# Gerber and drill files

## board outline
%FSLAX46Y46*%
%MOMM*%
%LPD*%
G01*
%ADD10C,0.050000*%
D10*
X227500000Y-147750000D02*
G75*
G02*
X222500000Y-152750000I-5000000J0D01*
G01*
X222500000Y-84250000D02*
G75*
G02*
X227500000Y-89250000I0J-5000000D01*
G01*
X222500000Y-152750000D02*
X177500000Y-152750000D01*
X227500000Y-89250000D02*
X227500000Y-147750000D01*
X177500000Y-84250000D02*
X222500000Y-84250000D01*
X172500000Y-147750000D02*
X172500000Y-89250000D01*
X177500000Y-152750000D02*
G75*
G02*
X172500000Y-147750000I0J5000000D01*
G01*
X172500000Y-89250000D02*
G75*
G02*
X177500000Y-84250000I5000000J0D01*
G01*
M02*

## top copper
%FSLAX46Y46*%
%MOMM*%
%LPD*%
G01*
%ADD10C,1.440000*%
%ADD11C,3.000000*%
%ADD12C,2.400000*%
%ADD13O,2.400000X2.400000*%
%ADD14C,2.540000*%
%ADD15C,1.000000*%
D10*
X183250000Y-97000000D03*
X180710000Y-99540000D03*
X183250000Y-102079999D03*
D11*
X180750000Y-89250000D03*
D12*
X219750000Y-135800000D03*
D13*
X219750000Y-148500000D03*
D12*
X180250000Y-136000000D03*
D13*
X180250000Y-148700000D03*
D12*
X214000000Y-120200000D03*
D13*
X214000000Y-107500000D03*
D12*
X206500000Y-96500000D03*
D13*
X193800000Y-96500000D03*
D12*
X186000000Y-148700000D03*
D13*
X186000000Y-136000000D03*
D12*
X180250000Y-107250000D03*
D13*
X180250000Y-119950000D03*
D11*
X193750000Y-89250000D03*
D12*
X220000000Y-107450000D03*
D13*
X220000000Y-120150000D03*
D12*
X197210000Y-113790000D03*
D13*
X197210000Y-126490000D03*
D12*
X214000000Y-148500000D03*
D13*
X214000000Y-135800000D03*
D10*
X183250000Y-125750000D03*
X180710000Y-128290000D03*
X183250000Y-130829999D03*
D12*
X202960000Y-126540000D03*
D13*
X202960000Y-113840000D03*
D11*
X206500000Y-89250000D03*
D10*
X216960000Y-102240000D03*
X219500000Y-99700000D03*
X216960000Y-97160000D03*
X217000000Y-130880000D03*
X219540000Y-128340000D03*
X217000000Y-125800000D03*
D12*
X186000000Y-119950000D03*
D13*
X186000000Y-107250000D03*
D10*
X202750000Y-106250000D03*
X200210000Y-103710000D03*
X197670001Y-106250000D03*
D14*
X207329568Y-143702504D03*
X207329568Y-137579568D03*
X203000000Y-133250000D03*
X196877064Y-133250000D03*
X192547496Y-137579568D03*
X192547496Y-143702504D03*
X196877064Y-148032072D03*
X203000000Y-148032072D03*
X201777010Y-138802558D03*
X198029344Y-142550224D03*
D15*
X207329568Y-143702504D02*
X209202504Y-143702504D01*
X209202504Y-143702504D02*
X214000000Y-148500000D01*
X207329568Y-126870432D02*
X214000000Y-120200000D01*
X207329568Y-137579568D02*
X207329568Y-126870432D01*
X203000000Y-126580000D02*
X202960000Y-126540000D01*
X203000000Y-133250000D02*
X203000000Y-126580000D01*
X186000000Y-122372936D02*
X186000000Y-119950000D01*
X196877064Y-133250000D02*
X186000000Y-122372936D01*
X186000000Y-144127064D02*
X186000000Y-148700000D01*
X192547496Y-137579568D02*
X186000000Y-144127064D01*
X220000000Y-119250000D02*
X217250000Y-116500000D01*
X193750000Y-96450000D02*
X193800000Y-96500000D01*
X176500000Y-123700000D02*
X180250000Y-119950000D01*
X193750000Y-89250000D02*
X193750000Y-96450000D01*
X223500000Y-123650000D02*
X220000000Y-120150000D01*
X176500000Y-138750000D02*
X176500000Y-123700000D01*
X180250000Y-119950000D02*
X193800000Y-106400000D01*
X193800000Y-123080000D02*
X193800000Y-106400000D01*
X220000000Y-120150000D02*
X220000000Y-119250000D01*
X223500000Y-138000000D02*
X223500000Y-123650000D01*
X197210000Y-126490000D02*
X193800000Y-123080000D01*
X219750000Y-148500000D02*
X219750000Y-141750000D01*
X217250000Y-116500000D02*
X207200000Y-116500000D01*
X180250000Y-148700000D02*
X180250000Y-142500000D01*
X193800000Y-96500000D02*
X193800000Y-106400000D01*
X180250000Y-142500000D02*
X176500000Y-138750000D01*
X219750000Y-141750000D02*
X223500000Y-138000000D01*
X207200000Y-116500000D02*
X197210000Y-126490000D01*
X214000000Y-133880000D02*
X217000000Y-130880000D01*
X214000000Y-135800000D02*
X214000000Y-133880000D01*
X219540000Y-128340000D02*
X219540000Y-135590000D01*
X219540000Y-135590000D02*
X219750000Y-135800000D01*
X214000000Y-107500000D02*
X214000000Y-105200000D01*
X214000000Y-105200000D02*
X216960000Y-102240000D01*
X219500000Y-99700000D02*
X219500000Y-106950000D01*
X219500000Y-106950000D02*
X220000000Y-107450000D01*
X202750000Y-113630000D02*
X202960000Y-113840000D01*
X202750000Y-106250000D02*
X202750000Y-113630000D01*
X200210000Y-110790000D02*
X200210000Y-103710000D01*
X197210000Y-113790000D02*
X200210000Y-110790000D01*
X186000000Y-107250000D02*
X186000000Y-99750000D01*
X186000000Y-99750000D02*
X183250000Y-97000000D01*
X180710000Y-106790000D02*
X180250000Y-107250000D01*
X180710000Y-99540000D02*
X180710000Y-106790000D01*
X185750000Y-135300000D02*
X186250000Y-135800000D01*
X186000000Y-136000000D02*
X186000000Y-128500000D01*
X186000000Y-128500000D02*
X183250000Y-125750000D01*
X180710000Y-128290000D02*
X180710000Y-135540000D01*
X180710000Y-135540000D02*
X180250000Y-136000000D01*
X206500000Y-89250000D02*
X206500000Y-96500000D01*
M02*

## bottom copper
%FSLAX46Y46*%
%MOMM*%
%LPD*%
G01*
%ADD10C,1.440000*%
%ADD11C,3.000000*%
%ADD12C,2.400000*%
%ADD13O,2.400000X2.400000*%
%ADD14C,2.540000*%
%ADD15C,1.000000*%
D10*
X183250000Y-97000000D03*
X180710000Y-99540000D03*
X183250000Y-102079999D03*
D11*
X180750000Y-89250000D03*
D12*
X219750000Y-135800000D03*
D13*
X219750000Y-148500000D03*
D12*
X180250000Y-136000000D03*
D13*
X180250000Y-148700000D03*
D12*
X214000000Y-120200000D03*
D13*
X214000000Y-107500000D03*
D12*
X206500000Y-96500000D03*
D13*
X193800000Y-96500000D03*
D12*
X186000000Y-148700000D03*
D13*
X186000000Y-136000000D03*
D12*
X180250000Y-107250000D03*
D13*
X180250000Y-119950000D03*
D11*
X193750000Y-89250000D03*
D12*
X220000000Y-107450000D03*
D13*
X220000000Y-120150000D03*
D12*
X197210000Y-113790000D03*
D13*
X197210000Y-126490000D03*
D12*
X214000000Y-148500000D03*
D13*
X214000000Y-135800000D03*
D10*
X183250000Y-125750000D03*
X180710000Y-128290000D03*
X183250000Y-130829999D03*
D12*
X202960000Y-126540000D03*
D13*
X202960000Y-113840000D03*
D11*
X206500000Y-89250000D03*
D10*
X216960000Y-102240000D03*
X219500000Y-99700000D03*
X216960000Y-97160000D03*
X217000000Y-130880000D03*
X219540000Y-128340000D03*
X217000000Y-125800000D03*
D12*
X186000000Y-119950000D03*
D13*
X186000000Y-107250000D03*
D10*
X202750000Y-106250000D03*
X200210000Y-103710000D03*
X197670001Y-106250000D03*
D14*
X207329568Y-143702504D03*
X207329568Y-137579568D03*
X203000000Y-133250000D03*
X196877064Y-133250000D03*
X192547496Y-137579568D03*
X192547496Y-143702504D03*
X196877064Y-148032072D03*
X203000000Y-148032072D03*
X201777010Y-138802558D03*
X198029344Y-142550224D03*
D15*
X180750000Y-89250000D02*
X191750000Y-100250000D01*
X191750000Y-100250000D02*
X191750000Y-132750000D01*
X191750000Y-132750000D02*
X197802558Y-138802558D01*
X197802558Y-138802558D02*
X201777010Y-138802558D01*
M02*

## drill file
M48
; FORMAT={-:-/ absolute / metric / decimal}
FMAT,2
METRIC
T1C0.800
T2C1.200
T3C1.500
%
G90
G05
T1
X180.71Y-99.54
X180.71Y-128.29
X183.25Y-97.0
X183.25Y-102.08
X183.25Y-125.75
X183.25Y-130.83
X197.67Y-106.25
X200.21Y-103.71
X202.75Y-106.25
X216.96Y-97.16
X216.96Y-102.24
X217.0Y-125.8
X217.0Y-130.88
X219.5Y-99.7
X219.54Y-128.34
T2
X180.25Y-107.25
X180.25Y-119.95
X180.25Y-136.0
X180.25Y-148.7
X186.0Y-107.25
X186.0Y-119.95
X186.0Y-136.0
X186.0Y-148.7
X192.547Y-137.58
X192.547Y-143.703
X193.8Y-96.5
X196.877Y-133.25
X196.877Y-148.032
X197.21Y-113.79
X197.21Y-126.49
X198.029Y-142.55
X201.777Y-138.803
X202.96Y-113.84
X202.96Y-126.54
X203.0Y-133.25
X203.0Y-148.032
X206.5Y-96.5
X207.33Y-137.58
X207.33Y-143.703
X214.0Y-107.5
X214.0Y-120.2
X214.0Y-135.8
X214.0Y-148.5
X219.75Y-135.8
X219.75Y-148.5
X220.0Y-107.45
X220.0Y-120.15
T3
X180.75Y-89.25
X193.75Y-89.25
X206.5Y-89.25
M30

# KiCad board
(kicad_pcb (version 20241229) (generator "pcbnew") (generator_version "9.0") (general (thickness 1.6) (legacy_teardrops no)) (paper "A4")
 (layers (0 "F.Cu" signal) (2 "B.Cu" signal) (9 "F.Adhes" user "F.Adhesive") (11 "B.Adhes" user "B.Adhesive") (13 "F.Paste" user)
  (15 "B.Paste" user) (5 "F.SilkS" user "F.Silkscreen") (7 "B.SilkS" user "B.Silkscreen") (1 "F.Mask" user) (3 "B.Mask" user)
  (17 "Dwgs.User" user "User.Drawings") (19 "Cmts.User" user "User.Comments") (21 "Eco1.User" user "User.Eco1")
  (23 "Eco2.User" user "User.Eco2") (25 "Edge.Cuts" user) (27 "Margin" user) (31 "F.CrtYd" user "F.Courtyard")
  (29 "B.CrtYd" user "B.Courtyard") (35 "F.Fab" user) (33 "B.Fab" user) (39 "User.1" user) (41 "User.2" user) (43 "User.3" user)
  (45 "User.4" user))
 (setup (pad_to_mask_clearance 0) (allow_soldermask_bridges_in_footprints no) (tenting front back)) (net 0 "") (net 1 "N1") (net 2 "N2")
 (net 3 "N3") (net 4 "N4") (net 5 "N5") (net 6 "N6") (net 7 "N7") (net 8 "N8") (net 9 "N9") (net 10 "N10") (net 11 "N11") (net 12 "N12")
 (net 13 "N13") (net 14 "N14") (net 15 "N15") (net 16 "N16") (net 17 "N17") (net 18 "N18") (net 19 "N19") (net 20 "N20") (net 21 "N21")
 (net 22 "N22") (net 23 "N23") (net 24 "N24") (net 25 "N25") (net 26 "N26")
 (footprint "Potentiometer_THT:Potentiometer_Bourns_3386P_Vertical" (layer "F.Cu") (at 183.25 97 180)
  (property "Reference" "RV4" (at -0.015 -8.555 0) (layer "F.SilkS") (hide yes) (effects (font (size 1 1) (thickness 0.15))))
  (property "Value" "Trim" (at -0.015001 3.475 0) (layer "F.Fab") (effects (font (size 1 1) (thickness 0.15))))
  (pad "1" thru_hole circle (at 0 0 180) (size 1.44 1.44) (drill 0.8) (layers "*.Cu" "*.Mask") (remove_unused_layers no) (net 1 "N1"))
  (pad "2" thru_hole circle (at 2.54 -2.54 180) (size 1.44 1.44) (drill 0.8) (layers "*.Cu" "*.Mask") (remove_unused_layers no) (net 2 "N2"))
  (pad "3" thru_hole circle (at 0 -5.079999 180) (size 1.44 1.44) (drill 0.8) (layers "*.Cu" "*.Mask") (remove_unused_layers no)
   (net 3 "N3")))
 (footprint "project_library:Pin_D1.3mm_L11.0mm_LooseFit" (layer "F.Cu") (at 180.75 89.25)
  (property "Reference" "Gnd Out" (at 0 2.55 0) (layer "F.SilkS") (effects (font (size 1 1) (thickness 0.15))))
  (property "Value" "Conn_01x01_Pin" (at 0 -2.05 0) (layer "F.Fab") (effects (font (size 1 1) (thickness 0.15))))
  (pad "1" thru_hole circle (at 0 0) (size 3 3) (drill 1.5) (layers "*.Cu" "*.Mask") (remove_unused_layers no) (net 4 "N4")))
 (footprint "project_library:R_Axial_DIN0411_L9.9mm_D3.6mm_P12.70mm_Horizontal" (layer "F.Cu") (at 219.75 135.8 -90)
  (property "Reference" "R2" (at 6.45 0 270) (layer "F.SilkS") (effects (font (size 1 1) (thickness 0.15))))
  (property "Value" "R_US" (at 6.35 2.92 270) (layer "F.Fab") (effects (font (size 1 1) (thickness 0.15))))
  (pad "1" thru_hole circle (at 0 0 270) (size 2.4 2.4) (drill 1.2) (layers "*.Cu" "*.Mask") (remove_unused_layers no) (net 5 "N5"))
  (pad "2" thru_hole oval (at 12.7 0 270) (size 2.4 2.4) (drill 1.2) (layers "*.Cu" "*.Mask") (remove_unused_layers no) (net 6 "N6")))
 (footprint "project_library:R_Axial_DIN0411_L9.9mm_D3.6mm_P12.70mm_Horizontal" (layer "F.Cu") (at 180.25 136 -90)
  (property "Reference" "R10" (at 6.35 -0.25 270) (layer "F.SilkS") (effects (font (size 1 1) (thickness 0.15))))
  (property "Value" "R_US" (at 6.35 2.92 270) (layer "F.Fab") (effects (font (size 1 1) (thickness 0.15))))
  (pad "1" thru_hole circle (at 0 0 270) (size 2.4 2.4) (drill 1.2) (layers "*.Cu" "*.Mask") (remove_unused_layers no) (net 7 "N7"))
  (pad "2" thru_hole oval (at 12.7 0 270) (size 2.4 2.4) (drill 1.2) (layers "*.Cu" "*.Mask") (remove_unused_layers no) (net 6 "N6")))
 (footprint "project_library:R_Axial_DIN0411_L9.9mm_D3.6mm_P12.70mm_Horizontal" (layer "F.Cu") (at 214 120.2 90)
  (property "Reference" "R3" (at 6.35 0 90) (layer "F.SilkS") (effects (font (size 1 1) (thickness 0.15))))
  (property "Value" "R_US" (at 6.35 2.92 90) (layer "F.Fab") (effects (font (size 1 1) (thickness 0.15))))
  (pad "1" thru_hole circle (at 0 0 90) (size 2.4 2.4) (drill 1.2) (layers "*.Cu" "*.Mask") (remove_unused_layers no) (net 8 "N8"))
  (pad "2" thru_hole oval (at 12.7 0 90) (size 2.4 2.4) (drill 1.2) (layers "*.Cu" "*.Mask") (remove_unused_layers no) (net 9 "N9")))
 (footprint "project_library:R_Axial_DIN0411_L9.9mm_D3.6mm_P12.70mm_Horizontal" (layer "F.Cu") (at 206.5 96.5 180)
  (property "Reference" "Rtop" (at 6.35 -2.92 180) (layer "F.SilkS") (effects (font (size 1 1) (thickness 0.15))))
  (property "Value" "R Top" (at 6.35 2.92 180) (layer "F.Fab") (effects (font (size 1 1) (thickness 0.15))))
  (pad "1" thru_hole circle (at 0 0 180) (size 2.4 2.4) (drill 1.2) (layers "*.Cu" "*.Mask") (remove_unused_layers no) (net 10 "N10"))
  (pad "2" thru_hole oval (at 12.7 0 180) (size 2.4 2.4) (drill 1.2) (layers "*.Cu" "*.Mask") (remove_unused_layers no) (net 6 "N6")))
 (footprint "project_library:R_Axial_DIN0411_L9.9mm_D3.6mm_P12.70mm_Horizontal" (layer "F.Cu") (at 186 148.7 90)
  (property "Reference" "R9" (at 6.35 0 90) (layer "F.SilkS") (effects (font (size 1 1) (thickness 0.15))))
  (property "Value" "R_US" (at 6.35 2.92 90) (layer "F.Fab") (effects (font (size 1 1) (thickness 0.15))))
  (pad "1" thru_hole circle (at 0 0 90) (size 2.4 2.4) (drill 1.2) (layers "*.Cu" "*.Mask") (remove_unused_layers no) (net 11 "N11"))
  (pad "2" thru_hole oval (at 12.7 0 90) (size 2.4 2.4) (drill 1.2) (layers "*.Cu" "*.Mask") (remove_unused_layers no) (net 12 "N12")))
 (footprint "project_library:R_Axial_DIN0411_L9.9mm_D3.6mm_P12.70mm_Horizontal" (layer "F.Cu") (at 180.25 107.25 -90)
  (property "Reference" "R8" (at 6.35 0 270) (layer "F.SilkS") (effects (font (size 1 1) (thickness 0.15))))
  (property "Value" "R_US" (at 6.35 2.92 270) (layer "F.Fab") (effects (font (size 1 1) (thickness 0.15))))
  (pad "1" thru_hole circle (at 0 0 270) (size 2.4 2.4) (drill 1.2) (layers "*.Cu" "*.Mask") (remove_unused_layers no) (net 2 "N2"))
  (pad "2" thru_hole oval (at 12.7 0 270) (size 2.4 2.4) (drill 1.2) (layers "*.Cu" "*.Mask") (remove_unused_layers no) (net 6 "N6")))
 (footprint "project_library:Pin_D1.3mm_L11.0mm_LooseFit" (layer "F.Cu") (at 193.75 89.25)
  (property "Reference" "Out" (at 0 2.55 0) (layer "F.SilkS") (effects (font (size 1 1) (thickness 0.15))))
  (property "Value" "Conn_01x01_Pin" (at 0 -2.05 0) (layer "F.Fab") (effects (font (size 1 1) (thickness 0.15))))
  (pad "1" thru_hole circle (at 0 0) (size 3 3) (drill 1.5) (layers "*.Cu" "*.Mask") (remove_unused_layers no) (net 6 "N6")))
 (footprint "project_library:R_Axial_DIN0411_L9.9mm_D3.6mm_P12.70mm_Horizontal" (layer "F.Cu") (at 220 107.45 -90)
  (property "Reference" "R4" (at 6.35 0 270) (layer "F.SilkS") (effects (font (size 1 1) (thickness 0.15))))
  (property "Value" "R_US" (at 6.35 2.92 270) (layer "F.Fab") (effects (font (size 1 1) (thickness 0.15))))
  (pad "1" thru_hole circle (at 0 0 270) (size 2.4 2.4) (drill 1.2) (layers "*.Cu" "*.Mask") (remove_unused_layers no) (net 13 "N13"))
  (pad "2" thru_hole oval (at 12.7 0 270) (size 2.4 2.4) (drill 1.2) (layers "*.Cu" "*.Mask") (remove_unused_layers no) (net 6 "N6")))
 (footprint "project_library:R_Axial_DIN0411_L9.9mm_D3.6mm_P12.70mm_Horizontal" (layer "F.Cu") (at 197.21 113.79 -90)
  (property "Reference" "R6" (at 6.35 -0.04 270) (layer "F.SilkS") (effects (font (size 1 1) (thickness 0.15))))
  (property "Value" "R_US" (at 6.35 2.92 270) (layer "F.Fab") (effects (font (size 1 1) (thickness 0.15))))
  (pad "1" thru_hole circle (at 0 0 270) (size 2.4 2.4) (drill 1.2) (layers "*.Cu" "*.Mask") (remove_unused_layers no) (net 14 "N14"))
  (pad "2" thru_hole oval (at 12.7 0 270) (size 2.4 2.4) (drill 1.2) (layers "*.Cu" "*.Mask") (remove_unused_layers no) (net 6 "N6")))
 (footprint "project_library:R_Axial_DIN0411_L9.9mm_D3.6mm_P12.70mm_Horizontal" (layer "F.Cu") (at 214 148.5 90)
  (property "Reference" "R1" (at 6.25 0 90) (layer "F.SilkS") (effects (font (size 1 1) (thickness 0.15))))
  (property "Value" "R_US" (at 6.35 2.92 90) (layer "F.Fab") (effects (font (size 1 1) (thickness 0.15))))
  (pad "1" thru_hole circle (at 0 0 90) (size 2.4 2.4) (drill 1.2) (layers "*.Cu" "*.Mask") (remove_unused_layers no) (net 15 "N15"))
  (pad "2" thru_hole oval (at 12.7 0 90) (size 2.4 2.4) (drill 1.2) (layers "*.Cu" "*.Mask") (remove_unused_layers no) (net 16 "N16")))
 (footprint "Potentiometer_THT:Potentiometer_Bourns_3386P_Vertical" (layer "F.Cu") (at 183.25 125.75 180)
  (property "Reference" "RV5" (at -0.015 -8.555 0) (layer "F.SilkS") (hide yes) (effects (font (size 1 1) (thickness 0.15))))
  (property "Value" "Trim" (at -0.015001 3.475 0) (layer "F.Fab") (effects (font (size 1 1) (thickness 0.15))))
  (pad "1" thru_hole circle (at 0 0 180) (size 1.44 1.44) (drill 0.8) (layers "*.Cu" "*.Mask") (remove_unused_layers no) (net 12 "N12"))
  (pad "2" thru_hole circle (at 2.54 -2.54 180) (size 1.44 1.44) (drill 0.8) (layers "*.Cu" "*.Mask") (remove_unused_layers no) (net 7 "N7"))
  (pad "3" thru_hole circle (at 0 -5.079999 180) (size 1.44 1.44) (drill 0.8) (layers "*.Cu" "*.Mask") (remove_unused_layers no)
   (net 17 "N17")))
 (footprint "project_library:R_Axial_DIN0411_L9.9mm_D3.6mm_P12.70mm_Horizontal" (layer "F.Cu") (at 202.96 126.54 90)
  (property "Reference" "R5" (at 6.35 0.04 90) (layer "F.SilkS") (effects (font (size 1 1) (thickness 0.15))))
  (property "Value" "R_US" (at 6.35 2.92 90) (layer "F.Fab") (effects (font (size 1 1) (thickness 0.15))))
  (pad "1" thru_hole circle (at 0 0 90) (size 2.4 2.4) (drill 1.2) (layers "*.Cu" "*.Mask") (remove_unused_layers no) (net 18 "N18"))
  (pad "2" thru_hole oval (at 12.7 0 90) (size 2.4 2.4) (drill 1.2) (layers "*.Cu" "*.Mask") (remove_unused_layers no) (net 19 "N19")))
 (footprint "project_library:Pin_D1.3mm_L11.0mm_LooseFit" (layer "F.Cu") (at 206.5 89.25)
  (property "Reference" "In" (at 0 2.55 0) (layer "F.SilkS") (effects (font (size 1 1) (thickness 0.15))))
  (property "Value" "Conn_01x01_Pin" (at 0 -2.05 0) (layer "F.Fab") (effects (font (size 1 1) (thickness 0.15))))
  (pad "1" thru_hole circle (at 0 0) (size 3 3) (drill 1.5) (layers "*.Cu" "*.Mask") (remove_unused_layers no) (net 10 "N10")))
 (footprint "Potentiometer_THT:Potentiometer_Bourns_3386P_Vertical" (layer "F.Cu") (at 216.96 102.24)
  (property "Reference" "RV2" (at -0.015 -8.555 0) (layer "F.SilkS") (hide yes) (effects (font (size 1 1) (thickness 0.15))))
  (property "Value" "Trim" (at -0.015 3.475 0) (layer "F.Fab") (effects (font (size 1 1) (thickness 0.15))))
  (pad "1" thru_hole circle (at 0 0) (size 1.44 1.44) (drill 0.8) (layers "*.Cu" "*.Mask") (remove_unused_layers no) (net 9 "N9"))
  (pad "2" thru_hole circle (at 2.54 -2.54) (size 1.44 1.44) (drill 0.8) (layers "*.Cu" "*.Mask") (remove_unused_layers no) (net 13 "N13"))
  (pad "3" thru_hole circle (at 0 -5.08) (size 1.44 1.44) (drill 0.8) (layers "*.Cu" "*.Mask") (remove_unused_layers no) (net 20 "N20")))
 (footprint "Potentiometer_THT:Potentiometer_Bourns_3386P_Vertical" (layer "F.Cu") (at 217 130.88)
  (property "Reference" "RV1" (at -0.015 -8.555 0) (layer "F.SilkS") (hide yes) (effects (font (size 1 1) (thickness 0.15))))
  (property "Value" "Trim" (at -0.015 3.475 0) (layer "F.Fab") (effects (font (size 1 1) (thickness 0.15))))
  (pad "1" thru_hole circle (at 0 0) (size 1.44 1.44) (drill 0.8) (layers "*.Cu" "*.Mask") (remove_unused_layers no) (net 16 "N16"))
  (pad "2" thru_hole circle (at 2.54 -2.54) (size 1.44 1.44) (drill 0.8) (layers "*.Cu" "*.Mask") (remove_unused_layers no) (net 5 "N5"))
  (pad "3" thru_hole circle (at 0 -5.08) (size 1.44 1.44) (drill 0.8) (layers "*.Cu" "*.Mask") (remove_unused_layers no) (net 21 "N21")))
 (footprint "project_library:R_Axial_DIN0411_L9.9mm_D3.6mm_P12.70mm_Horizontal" (layer "F.Cu") (at 186 119.95 90)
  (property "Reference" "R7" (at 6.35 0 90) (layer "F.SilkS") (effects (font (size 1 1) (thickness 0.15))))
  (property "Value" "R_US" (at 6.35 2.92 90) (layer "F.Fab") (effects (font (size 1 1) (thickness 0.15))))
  (pad "1" thru_hole circle (at 0 0 90) (size 2.4 2.4) (drill 1.2) (layers "*.Cu" "*.Mask") (remove_unused_layers no) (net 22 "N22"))
  (pad "2" thru_hole oval (at 12.7 0 90) (size 2.4 2.4) (drill 1.2) (layers "*.Cu" "*.Mask") (remove_unused_layers no) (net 1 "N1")))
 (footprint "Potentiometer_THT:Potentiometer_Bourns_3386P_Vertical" (layer "F.Cu") (at 202.75 106.25 90)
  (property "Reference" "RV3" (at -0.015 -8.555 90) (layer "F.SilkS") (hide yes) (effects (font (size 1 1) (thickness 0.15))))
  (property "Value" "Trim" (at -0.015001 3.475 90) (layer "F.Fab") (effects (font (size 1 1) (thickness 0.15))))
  (pad "1" thru_hole circle (at 0 0 90) (size 1.44 1.44) (drill 0.8) (layers "*.Cu" "*.Mask") (remove_unused_layers no) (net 19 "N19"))
  (pad "2" thru_hole circle (at 2.54 -2.54 90) (size 1.44 1.44) (drill 0.8) (layers "*.Cu" "*.Mask") (remove_unused_layers no)
   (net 14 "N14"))
  (pad "3" thru_hole circle (at 0 -5.079999 90) (size 1.44 1.44) (drill 0.8) (layers "*.Cu" "*.Mask") (remove_unused_layers no)
   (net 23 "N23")))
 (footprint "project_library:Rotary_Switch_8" (layer "B.Cu") (at 199.938532 140.641036 45)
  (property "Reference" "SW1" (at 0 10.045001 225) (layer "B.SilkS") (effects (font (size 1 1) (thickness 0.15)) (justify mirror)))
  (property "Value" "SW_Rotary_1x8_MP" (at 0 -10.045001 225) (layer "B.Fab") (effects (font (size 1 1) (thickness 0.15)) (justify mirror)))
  (pad "1" thru_hole circle (at 3.061467 7.391036 22.5) (size 2.54 2.54) (drill 1.2) (layers "*.Cu" "*.Mask") (remove_unused_layers no)
   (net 15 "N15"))
  (pad "2" thru_hole circle (at 7.391036 3.061467 22.5) (size 2.54 2.54) (drill 1.2) (layers "*.Cu" "*.Mask") (remove_unused_layers no)
   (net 8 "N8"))
  (pad "3" thru_hole circle (at 7.391036 -3.061467 22.5) (size 2.54 2.54) (drill 1.2) (layers "*.Cu" "*.Mask") (remove_unused_layers no)
   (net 18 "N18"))
  (pad "4" thru_hole circle (at 3.061467 -7.391036 22.5) (size 2.54 2.54) (drill 1.2) (layers "*.Cu" "*.Mask") (remove_unused_layers no)
   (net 22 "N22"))
  (pad "5" thru_hole circle (at -3.061467 -7.391036 22.5) (size 2.54 2.54) (drill 1.2) (layers "*.Cu" "*.Mask") (remove_unused_layers no)
   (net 11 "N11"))
  (pad "6" thru_hole circle (at -7.391036 -3.061467 22.5) (size 2.54 2.54) (drill 1.2) (layers "*.Cu" "*.Mask") (remove_unused_layers no)
   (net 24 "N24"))
  (pad "7" thru_hole circle (at -7.391036 3.061467 22.5) (size 2.54 2.54) (drill 1.2) (layers "*.Cu" "*.Mask") (remove_unused_layers no)
   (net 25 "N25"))
  (pad "8" thru_hole circle (at -3.061467 7.391036 22.5) (size 2.54 2.54) (drill 1.2) (layers "*.Cu" "*.Mask") (remove_unused_layers no)
   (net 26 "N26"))
  (pad "9" thru_hole circle (at 2.600001 0 45) (size 2.54 2.54) (drill 1.2) (layers "*.Cu" "*.Mask") (remove_unused_layers no) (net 4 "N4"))
  (pad "MP" thru_hole circle (at -2.7 0 45) (size 2.54 2.54) (drill 1.2) (layers "*.Cu" "*.Mask") (remove_unused_layers no)))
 (gr_arc (start 227.5 147.75) (mid 226.035534 151.285534) (end 222.5 152.75) (stroke (width 0.05) (type default)) (layer "Edge.Cuts"))
 (gr_arc (start 222.5 84.25) (mid 226.035534 85.714466) (end 227.5 89.25) (stroke (width 0.05) (type default)) (layer "Edge.Cuts"))
 (gr_line (start 222.5 152.75) (end 177.5 152.75) (stroke (width 0.05) (type default)) (layer "Edge.Cuts"))
 (gr_line (start 227.5 89.25) (end 227.5 147.75) (stroke (width 0.05) (type default)) (layer "Edge.Cuts"))
 (gr_line (start 177.5 84.25) (end 222.5 84.25) (stroke (width 0.05) (type default)) (layer "Edge.Cuts"))
 (gr_line (start 172.5 147.75) (end 172.5 89.25) (stroke (width 0.05) (type default)) (layer "Edge.Cuts"))
 (gr_arc (start 177.5 152.75) (mid 173.964466 151.285534) (end 172.5 147.75) (stroke (width 0.05) (type default)) (layer "Edge.Cuts"))
 (gr_arc (start 172.5 89.25) (mid 173.964466 85.714466) (end 177.5 84.25) (stroke (width 0.05) (type default)) (layer "Edge.Cuts"))
 (segment (start 207.329568 143.702504) (end 209.202504 143.702504) (width 1) (layer "F.Cu") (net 15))
 (segment (start 209.202504 143.702504) (end 214 148.5) (width 1) (layer "F.Cu") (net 15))
 (segment (start 207.329568 126.870432) (end 214 120.2) (width 1) (layer "F.Cu") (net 8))
 (segment (start 207.329568 137.579568) (end 207.329568 126.870432) (width 1) (layer "F.Cu") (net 8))
 (segment (start 203 126.58) (end 202.96 126.54) (width 1) (layer "F.Cu") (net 18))
 (segment (start 203 133.25) (end 203 126.58) (width 1) (layer "F.Cu") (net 18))
 (segment (start 186 122.372936) (end 186 119.95) (width 1) (layer "F.Cu") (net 22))
 (segment (start 196.877064 133.25) (end 186 122.372936) (width 1) (layer "F.Cu") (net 22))
 (segment (start 186 144.127064) (end 186 148.7) (width 1) (layer "F.Cu") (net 11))
 (segment (start 192.547496 137.579568) (end 186 144.127064) (width 1) (layer "F.Cu") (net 11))
 (segment (start 220 119.25) (end 217.25 116.5) (width 1) (layer "F.Cu") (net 6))
 (segment (start 193.75 96.45) (end 193.8 96.5) (width 1) (layer "F.Cu") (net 6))
 (segment (start 176.5 123.7) (end 180.25 119.95) (width 1) (layer "F.Cu") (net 6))
 (segment (start 193.75 89.25) (end 193.75 96.45) (width 1) (layer "F.Cu") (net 6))
 (segment (start 223.5 123.65) (end 220 120.15) (width 1) (layer "F.Cu") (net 6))
 (segment (start 176.5 138.75) (end 176.5 123.7) (width 1) (layer "F.Cu") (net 6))
 (segment (start 180.25 119.95) (end 193.8 106.4) (width 1) (layer "F.Cu") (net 6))
 (segment (start 193.8 123.08) (end 193.8 106.4) (width 1) (layer "F.Cu") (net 6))
 (segment (start 220 120.15) (end 220 119.25) (width 1) (layer "F.Cu") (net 6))
 (segment (start 223.5 138) (end 223.5 123.65) (width 1) (layer "F.Cu") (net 6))
 (segment (start 197.21 126.49) (end 193.8 123.08) (width 1) (layer "F.Cu") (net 6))
 (segment (start 219.75 148.5) (end 219.75 141.75) (width 1) (layer "F.Cu") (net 6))
 (segment (start 217.25 116.5) (end 207.2 116.5) (width 1) (layer "F.Cu") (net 6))
 (segment (start 180.25 148.7) (end 180.25 142.5) (width 1) (layer "F.Cu") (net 6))
 (segment (start 193.8 96.5) (end 193.8 106.4) (width 1) (layer "F.Cu") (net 6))
 (segment (start 180.25 142.5) (end 176.5 138.75) (width 1) (layer "F.Cu") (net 6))
 (segment (start 219.75 141.75) (end 223.5 138) (width 1) (layer "F.Cu") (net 6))
 (segment (start 207.2 116.5) (end 197.21 126.49) (width 1) (layer "F.Cu") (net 6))
 (segment (start 214 133.88) (end 217 130.88) (width 1) (layer "F.Cu") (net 16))
 (segment (start 214 135.8) (end 214 133.88) (width 1) (layer "F.Cu") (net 16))
 (segment (start 219.54 128.34) (end 219.54 135.59) (width 1) (layer "F.Cu") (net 5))
 (segment (start 219.54 135.59) (end 219.75 135.8) (width 1) (layer "F.Cu") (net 5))
 (segment (start 214 107.5) (end 214 105.2) (width 1) (layer "F.Cu") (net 9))
 (segment (start 214 105.2) (end 216.96 102.24) (width 1) (layer "F.Cu") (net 9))
 (segment (start 219.5 99.7) (end 219.5 106.95) (width 1) (layer "F.Cu") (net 13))
 (segment (start 219.5 106.95) (end 220 107.45) (width 1) (layer "F.Cu") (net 13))
 (segment (start 202.75 113.63) (end 202.96 113.84) (width 1) (layer "F.Cu") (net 19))
 (segment (start 202.75 106.25) (end 202.75 113.63) (width 1) (layer "F.Cu") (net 19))
 (segment (start 200.21 110.79) (end 200.21 103.71) (width 1) (layer "F.Cu") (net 14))
 (segment (start 197.21 113.79) (end 200.21 110.79) (width 1) (layer "F.Cu") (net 14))
 (segment (start 186 107.25) (end 186 99.75) (width 1) (layer "F.Cu") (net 1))
 (segment (start 186 99.75) (end 183.25 97) (width 1) (layer "F.Cu") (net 1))
 (segment (start 180.71 106.79) (end 180.25 107.25) (width 1) (layer "F.Cu") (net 2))
 (segment (start 180.71 99.54) (end 180.71 106.79) (width 1) (layer "F.Cu") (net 2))
 (segment (start 185.75 135.3) (end 186.25 135.8) (width 1) (layer "F.Cu") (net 12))
 (segment (start 186 136) (end 186 128.5) (width 1) (layer "F.Cu") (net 12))
 (segment (start 186 128.5) (end 183.25 125.75) (width 1) (layer "F.Cu") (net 12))
 (segment (start 180.71 128.29) (end 180.71 135.54) (width 1) (layer "F.Cu") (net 7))
 (segment (start 180.71 135.54) (end 180.25 136) (width 1) (layer "F.Cu") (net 7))
 (segment (start 206.5 89.25) (end 206.5 96.5) (width 1) (layer "F.Cu") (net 10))
 (segment (start 180.75 89.25) (end 191.75 100.25) (width 1) (layer "B.Cu") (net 4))
 (segment (start 191.75 100.25) (end 191.75 132.75) (width 1) (layer "B.Cu") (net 4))
 (segment (start 191.75 132.75) (end 197.802558 138.802558) (width 1) (layer "B.Cu") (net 4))
 (segment (start 197.802558 138.802558) (end 201.77701 138.802558) (width 1) (layer "B.Cu") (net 4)))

